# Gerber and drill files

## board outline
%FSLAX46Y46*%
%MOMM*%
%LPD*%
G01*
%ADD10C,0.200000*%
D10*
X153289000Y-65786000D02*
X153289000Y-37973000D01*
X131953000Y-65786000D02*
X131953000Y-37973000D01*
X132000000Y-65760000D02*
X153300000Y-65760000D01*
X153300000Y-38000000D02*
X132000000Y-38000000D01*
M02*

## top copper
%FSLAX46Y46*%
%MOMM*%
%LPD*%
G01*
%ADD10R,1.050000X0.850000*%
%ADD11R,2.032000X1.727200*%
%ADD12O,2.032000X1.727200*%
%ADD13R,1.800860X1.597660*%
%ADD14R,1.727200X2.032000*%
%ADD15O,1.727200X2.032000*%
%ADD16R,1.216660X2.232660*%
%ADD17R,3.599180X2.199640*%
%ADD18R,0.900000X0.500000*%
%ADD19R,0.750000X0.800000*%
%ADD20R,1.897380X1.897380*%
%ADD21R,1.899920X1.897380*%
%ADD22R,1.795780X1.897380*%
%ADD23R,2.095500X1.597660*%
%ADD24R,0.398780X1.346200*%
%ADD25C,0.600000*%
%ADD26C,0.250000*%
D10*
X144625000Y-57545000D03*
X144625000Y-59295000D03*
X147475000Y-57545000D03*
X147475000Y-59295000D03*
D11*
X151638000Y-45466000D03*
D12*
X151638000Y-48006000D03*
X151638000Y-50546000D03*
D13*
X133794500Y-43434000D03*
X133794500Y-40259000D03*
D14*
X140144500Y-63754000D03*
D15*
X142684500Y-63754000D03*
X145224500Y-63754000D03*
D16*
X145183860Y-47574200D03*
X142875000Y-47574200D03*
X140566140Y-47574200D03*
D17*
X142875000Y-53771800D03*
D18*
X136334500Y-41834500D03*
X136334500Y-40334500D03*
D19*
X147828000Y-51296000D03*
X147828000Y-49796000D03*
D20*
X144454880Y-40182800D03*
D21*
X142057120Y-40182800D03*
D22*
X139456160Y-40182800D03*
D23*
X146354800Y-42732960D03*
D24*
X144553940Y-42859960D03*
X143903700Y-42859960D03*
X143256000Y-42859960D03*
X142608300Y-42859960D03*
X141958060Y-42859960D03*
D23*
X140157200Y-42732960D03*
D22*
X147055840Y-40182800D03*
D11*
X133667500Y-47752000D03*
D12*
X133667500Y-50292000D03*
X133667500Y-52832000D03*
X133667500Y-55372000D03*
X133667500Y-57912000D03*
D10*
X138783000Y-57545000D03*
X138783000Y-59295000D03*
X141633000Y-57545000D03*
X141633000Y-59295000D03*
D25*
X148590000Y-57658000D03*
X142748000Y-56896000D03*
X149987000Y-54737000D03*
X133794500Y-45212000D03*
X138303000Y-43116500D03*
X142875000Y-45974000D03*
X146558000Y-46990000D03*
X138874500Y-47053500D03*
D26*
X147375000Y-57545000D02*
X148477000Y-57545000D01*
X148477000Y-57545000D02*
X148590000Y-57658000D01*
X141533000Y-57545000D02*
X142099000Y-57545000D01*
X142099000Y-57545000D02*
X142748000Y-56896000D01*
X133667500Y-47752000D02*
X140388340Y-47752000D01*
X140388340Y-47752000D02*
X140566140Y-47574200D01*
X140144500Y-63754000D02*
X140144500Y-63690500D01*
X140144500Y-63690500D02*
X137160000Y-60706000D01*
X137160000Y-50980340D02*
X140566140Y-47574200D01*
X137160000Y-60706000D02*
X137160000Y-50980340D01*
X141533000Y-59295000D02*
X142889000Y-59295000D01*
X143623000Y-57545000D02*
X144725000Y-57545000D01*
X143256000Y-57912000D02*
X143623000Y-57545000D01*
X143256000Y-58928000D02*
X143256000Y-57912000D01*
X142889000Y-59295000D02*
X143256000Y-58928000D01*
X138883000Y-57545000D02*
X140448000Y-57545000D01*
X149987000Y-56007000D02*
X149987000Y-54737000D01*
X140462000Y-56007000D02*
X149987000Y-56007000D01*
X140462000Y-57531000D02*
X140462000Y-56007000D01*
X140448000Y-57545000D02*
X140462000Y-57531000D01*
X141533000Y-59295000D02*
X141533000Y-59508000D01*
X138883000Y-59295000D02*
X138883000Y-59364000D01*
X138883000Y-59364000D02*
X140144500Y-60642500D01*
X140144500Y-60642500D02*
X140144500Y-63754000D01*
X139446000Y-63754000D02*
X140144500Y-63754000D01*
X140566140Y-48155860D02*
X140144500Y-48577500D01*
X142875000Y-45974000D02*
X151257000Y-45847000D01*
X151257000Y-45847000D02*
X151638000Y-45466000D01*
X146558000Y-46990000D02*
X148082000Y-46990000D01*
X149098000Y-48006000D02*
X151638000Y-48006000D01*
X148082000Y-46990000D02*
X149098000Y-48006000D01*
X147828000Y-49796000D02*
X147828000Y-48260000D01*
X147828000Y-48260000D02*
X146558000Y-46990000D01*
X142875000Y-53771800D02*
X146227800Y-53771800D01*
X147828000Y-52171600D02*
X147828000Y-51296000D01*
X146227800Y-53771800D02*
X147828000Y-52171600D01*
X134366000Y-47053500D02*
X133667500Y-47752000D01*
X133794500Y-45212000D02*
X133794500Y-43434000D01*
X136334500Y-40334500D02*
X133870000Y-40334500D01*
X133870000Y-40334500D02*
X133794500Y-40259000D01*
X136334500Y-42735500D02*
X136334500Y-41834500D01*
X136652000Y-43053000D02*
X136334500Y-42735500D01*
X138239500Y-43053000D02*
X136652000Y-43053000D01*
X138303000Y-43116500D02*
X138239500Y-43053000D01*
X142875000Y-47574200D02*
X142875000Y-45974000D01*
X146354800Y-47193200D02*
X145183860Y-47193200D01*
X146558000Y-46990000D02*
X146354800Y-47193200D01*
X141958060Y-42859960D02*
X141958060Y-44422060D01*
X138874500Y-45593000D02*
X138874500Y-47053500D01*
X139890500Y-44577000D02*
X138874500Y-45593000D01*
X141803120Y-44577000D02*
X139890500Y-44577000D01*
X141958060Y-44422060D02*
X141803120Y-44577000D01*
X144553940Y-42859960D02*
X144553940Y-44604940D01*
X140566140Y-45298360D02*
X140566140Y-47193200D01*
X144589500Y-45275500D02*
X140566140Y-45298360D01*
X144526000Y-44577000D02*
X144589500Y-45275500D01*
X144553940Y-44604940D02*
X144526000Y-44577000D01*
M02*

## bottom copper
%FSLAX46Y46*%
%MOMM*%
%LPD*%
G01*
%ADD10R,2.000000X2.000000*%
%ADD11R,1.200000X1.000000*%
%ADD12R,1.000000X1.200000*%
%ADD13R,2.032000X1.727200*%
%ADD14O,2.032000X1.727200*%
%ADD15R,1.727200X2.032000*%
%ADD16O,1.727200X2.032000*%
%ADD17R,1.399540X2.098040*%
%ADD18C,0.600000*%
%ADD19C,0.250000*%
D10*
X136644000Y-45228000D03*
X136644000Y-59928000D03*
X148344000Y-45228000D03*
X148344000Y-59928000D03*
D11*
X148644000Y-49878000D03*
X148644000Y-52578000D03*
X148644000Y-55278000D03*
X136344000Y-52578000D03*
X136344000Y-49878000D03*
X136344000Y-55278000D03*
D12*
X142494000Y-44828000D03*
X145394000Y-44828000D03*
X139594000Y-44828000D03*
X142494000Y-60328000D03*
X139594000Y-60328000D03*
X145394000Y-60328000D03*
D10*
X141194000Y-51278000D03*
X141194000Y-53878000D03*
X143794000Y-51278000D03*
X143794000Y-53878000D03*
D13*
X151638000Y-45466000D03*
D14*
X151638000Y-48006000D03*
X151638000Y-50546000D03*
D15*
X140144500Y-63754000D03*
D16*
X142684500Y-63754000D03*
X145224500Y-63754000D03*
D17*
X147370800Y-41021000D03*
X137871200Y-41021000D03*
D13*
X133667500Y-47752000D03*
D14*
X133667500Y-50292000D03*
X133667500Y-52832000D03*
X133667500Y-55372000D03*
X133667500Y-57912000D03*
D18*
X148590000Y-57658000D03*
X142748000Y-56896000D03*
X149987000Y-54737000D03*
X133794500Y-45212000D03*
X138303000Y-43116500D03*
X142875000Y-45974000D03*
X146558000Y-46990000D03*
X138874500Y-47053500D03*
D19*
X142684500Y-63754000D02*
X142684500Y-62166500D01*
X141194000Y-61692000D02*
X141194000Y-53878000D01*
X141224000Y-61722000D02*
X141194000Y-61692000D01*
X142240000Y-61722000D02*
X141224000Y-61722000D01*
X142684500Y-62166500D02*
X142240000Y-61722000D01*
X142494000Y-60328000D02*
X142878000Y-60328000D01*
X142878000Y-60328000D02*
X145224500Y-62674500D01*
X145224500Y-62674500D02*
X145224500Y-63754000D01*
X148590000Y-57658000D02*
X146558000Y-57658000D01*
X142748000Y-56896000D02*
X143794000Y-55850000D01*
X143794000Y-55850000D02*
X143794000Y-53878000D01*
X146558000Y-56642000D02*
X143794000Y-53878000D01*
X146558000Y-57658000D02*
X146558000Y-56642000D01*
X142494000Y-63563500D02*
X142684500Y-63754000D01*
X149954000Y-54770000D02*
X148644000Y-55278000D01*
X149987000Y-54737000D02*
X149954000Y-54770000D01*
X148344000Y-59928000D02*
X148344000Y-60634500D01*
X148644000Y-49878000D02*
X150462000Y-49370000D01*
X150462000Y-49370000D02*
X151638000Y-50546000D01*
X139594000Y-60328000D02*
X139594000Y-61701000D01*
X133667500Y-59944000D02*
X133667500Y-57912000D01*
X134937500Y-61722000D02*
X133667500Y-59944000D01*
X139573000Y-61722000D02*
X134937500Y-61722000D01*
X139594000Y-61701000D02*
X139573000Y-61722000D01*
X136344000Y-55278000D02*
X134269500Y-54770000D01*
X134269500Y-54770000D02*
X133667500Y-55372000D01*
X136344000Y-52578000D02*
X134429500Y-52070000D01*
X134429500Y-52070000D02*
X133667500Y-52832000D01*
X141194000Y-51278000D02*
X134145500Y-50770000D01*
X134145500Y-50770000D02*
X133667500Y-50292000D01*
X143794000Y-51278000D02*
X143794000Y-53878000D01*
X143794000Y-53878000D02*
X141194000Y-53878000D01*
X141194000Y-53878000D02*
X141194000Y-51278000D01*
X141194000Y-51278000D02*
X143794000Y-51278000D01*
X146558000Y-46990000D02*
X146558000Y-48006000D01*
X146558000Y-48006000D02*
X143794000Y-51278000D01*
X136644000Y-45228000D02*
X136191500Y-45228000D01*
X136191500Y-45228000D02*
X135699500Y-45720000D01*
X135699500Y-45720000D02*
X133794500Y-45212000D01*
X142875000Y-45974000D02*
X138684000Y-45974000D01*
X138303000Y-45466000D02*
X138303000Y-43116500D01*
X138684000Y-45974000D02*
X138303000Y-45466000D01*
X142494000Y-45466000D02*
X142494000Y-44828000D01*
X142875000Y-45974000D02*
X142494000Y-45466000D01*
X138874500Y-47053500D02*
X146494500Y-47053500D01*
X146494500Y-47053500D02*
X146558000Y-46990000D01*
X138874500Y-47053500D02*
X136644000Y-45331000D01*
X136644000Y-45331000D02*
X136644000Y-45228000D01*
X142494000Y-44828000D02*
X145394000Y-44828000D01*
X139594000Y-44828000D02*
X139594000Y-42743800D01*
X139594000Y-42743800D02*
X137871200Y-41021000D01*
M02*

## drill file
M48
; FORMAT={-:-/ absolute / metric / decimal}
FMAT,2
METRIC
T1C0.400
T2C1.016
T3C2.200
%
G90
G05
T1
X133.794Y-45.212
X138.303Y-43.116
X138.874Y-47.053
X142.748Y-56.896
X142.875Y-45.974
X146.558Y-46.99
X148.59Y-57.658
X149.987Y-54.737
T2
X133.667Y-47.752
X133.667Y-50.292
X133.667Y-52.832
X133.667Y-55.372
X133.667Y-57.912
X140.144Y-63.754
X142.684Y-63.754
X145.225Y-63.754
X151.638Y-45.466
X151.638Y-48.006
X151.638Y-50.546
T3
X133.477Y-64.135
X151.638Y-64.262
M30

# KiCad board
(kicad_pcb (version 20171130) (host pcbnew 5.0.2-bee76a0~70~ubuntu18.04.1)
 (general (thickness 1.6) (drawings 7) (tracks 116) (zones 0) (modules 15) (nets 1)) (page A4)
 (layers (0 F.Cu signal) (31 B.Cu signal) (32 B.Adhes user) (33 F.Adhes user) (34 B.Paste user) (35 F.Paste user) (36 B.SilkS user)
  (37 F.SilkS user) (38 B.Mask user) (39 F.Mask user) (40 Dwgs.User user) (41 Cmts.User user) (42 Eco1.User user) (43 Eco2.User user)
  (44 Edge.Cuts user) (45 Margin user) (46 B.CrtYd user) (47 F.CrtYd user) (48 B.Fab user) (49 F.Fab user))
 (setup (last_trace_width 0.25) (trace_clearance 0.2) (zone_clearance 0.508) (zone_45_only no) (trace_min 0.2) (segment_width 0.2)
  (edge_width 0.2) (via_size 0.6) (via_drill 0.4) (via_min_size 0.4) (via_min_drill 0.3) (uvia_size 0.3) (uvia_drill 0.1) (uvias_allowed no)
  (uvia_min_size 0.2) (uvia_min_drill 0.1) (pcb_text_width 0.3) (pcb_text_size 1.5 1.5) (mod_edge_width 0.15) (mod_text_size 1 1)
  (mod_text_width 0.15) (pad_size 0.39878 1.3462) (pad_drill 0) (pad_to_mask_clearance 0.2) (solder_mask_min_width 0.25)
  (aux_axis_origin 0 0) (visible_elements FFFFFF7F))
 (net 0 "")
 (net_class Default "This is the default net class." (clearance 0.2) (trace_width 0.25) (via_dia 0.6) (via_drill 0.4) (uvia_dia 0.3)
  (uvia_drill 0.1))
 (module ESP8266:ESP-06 (layer B.Cu) (at 142.494 52.578 270)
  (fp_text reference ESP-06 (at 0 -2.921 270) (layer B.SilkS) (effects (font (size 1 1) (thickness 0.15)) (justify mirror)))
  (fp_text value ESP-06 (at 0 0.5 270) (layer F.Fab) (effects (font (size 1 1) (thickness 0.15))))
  (pad GND smd rect (at -7.35 5.85 270) (size 2 2) (layers B.Cu B.Paste B.Mask))
  (pad GP5 smd rect (at 7.35 5.85 270) (size 2 2) (layers B.Cu B.Paste B.Mask))
  (pad GP16 smd rect (at -7.35 -5.85 270) (size 2 2) (layers B.Cu B.Paste B.Mask))
  (pad GP15 smd rect (at 7.35 -5.85 270) (size 2 2) (layers B.Cu B.Paste B.Mask))
  (pad GP14 smd rect (at -2.7 -6.15 270) (size 1 1.2) (layers B.Cu B.Paste B.Mask))
  (pad GP12 smd rect (at 0 -6.15 270) (size 1 1.2) (layers B.Cu B.Paste B.Mask))
  (pad GP13 smd rect (at 2.7 -6.15 270) (size 1 1.2) (layers B.Cu B.Paste B.Mask))
  (pad TX smd rect (at 0 6.15 270) (size 1 1.2) (layers B.Cu B.Paste B.Mask))
  (pad RST smd rect (at -2.7 6.15 270) (size 1 1.2) (layers B.Cu B.Paste B.Mask))
  (pad RX smd rect (at 2.7 6.15 270) (size 1 1.2) (layers B.Cu B.Paste B.Mask))
  (pad 3.3 smd rect (at -7.75 0 270) (size 1.2 1) (layers B.Cu B.Paste B.Mask))
  (pad CHPD smd rect (at -7.75 -2.9 270) (size 1.2 1) (layers B.Cu B.Paste B.Mask))
  (pad ANT smd rect (at -7.75 2.9 270) (size 1.2 1) (layers B.Cu B.Paste B.Mask))
  (pad GP2 smd rect (at 7.75 0 270) (size 1.2 1) (layers B.Cu B.Paste B.Mask))
  (pad GP0 smd rect (at 7.75 2.9 270) (size 1.2 1) (layers B.Cu B.Paste B.Mask))
  (pad GP4 smd rect (at 7.75 -2.9 270) (size 1.2 1) (layers B.Cu B.Paste B.Mask))
  (pad GND smd rect (at -1.3 1.3 270) (size 2 2) (layers B.Cu B.Paste B.Mask))
  (pad GND smd rect (at 1.3 1.3 270) (size 2 2) (layers B.Cu B.Paste B.Mask))
  (pad GND smd rect (at -1.3 -1.3 270) (size 2 2) (layers B.Cu B.Paste B.Mask))
  (pad GND smd rect (at 1.3 -1.3 270) (size 2 2) (layers B.Cu B.Paste B.Mask)))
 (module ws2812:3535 (layer F.Cu) (at 146.05 58.42 180)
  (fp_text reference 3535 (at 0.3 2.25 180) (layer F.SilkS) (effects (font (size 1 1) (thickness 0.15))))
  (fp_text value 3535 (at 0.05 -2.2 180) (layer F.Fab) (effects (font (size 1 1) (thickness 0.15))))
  (pad IN smd rect (at 1.325 0.875 180) (size 1.05 0.85) (drill (offset 0.1 0)) (layers F.Cu F.Paste F.Mask))
  (pad VDD smd rect (at 1.325 -0.875 180) (size 1.05 0.85) (drill (offset 0.1 0)) (layers F.Cu F.Paste F.Mask))
  (pad VSS smd rect (at -1.325 0.875 180) (size 1.05 0.85) (drill (offset -0.1 0)) (layers F.Cu F.Paste F.Mask))
  (pad OUT smd rect (at -1.325 -0.875 180) (size 1.05 0.85) (drill (offset -0.1 0)) (layers F.Cu F.Paste F.Mask)))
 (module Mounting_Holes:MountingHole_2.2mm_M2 (layer F.Cu) (at 133.477 64.135)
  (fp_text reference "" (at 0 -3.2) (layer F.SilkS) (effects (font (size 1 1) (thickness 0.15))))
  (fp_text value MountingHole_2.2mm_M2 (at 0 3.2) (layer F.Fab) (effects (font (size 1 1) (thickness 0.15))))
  (pad 1 np_thru_hole circle (at 0 0) (size 2.2 2.2) (drill 2.2) (layers *.Cu *.Mask F.SilkS)))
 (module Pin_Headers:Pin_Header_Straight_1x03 (layer F.Cu) (at 151.638 45.466)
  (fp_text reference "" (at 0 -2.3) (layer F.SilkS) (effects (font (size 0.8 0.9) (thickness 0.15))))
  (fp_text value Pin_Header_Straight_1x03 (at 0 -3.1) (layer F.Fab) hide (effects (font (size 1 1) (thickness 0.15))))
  (pad 1 thru_hole rect (at 0 0) (size 2.032 1.7272) (drill 1.016) (layers *.Cu *.Mask F.SilkS))
  (pad 2 thru_hole oval (at 0 2.54) (size 2.032 1.7272) (drill 1.016) (layers *.Cu *.Mask F.SilkS))
  (pad 3 thru_hole oval (at 0 5.08) (size 2.032 1.7272) (drill 1.016) (layers *.Cu *.Mask F.SilkS)))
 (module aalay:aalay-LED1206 (layer F.Cu) (at 133.7945 41.8465 90)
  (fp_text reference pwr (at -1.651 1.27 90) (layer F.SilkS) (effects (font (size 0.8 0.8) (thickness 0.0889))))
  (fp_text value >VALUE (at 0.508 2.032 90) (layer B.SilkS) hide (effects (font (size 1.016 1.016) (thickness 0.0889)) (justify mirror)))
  (pad A smd rect (at -1.5875 0 90) (size 1.59766 1.80086) (layers F.Cu F.Paste F.Mask))
  (pad K smd rect (at 1.5875 0 90) (size 1.59766 1.80086) (layers F.Cu F.Paste F.Mask)))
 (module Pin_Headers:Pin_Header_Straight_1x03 (layer F.Cu) (at 140.1445 63.754 90)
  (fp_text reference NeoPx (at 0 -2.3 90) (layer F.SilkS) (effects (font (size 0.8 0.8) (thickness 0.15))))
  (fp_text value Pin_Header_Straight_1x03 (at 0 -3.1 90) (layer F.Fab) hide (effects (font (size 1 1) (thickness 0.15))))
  (pad 1 thru_hole rect (at 0 0 90) (size 2.032 1.7272) (drill 1.016) (layers *.Cu *.Mask F.SilkS))
  (pad 2 thru_hole oval (at 0 2.54 90) (size 2.032 1.7272) (drill 1.016) (layers *.Cu *.Mask F.SilkS))
  (pad 3 thru_hole oval (at 0 5.08 90) (size 2.032 1.7272) (drill 1.016) (layers *.Cu *.Mask F.SilkS)))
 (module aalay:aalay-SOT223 (layer F.Cu) (at 142.875 50.673 180)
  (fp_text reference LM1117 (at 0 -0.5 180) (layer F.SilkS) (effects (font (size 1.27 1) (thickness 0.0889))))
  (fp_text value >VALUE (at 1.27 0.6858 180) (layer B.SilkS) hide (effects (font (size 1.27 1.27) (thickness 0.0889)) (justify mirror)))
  (pad GND smd rect (at -2.30886 3.0988 180) (size 1.21666 2.23266) (layers F.Cu F.Paste F.Mask))
  (pad OUT smd rect (at 0 3.0988 180) (size 1.21666 2.23266) (layers F.Cu F.Paste F.Mask))
  (pad IN smd rect (at 2.30886 3.0988 180) (size 1.21666 2.23266) (layers F.Cu F.Paste F.Mask))
  (pad OUT smd rect (at 0 -3.0988 180) (size 3.59918 2.19964) (layers F.Cu F.Paste F.Mask)))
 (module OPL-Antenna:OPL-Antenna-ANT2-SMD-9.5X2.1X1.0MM (layer B.Cu) (at 142.621 41.021 180)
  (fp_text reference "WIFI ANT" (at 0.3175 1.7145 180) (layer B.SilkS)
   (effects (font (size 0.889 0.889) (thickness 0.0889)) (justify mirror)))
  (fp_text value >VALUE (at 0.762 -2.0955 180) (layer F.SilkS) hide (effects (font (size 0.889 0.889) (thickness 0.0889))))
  (pad 1 smd rect (at -4.7498 0 180) (size 1.39954 2.09804) (layers B.Cu B.Paste B.Mask))
  (pad 2 smd rect (at 4.7498 0 180) (size 1.39954 2.09804) (layers B.Cu B.Paste B.Mask)))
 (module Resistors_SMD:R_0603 (layer F.Cu) (at 136.3345 41.0845 90)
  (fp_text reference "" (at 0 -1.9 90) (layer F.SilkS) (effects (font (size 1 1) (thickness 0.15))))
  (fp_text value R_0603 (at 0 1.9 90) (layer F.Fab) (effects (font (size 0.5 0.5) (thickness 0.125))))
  (pad 1 smd rect (at -0.75 0 90) (size 0.5 0.9) (layers F.Cu F.Paste F.Mask))
  (pad 2 smd rect (at 0.75 0 90) (size 0.5 0.9) (layers F.Cu F.Paste F.Mask)))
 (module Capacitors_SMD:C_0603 (layer F.Cu) (at 147.828 50.546 90)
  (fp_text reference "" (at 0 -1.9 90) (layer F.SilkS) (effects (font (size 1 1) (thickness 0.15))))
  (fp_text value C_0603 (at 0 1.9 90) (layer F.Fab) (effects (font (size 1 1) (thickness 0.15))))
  (pad 1 smd rect (at -0.75 0 90) (size 0.8 0.75) (layers F.Cu F.Paste F.Mask))
  (pad 2 smd rect (at 0.75 0 90) (size 0.8 0.75) (layers F.Cu F.Paste F.Mask)))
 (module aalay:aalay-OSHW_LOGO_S (layer F.Cu) (at 150.622 39.878)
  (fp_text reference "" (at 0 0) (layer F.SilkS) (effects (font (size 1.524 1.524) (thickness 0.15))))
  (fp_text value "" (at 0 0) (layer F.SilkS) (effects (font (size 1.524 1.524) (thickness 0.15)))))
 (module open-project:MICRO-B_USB (layer F.Cu) (at 143.256 38.735 180)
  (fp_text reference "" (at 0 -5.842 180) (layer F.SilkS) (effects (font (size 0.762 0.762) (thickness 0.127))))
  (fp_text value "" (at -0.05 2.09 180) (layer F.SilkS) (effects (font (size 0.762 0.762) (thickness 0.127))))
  (pad "" smd rect (at -1.19888 -1.4478 180) (size 1.89738 1.89738) (layers F.Cu F.Paste F.Mask))
  (pad "" smd rect (at 1.19888 -1.4478 180) (size 1.89992 1.89738) (layers F.Cu F.Paste F.Mask))
  (pad "" smd rect (at 3.79984 -1.4478 180) (size 1.79578 1.89738) (layers F.Cu F.Paste F.Mask))
  (pad "" smd rect (at -3.0988 -3.99796 180) (size 2.0955 1.59766) (layers F.Cu F.Paste F.Mask))
  (pad +5 smd rect (at -1.29794 -4.12496 180) (size 0.39878 1.3462) (layers F.Cu F.Paste F.Mask) (clearance 0.2032))
  (pad 2 smd rect (at -0.6477 -4.12496 180) (size 0.39878 1.3462) (layers F.Cu F.Paste F.Mask) (clearance 0.2032))
  (pad 3 smd rect (at 0 -4.12496 180) (size 0.39878 1.3462) (layers F.Cu F.Paste F.Mask) (clearance 0.2032))
  (pad 4 smd rect (at 0.6477 -4.12496 180) (size 0.39878 1.3462) (layers F.Cu F.Paste F.Mask) (clearance 0.2032))
  (pad GND smd rect (at 1.29794 -4.12496 180) (size 0.39878 1.3462) (layers F.Cu F.Paste F.Mask) (clearance 0.2032))
  (pad "" smd rect (at 3.0988 -3.99796 180) (size 2.0955 1.59766) (layers F.Cu F.Paste F.Mask))
  (pad "" smd rect (at -3.79984 -1.4478 180) (size 1.79578 1.89738) (layers F.Cu F.Paste F.Mask)))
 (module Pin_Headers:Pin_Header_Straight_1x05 (layer F.Cu) (at 133.6675 47.752)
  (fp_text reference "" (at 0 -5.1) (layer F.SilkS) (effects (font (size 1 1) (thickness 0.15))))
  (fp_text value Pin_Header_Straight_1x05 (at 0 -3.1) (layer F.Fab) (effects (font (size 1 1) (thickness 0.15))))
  (pad 1 thru_hole rect (at 0 0) (size 2.032 1.7272) (drill 1.016) (layers *.Cu *.Mask F.SilkS))
  (pad 2 thru_hole oval (at 0 2.54) (size 2.032 1.7272) (drill 1.016) (layers *.Cu *.Mask F.SilkS))
  (pad 3 thru_hole oval (at 0 5.08) (size 2.032 1.7272) (drill 1.016) (layers *.Cu *.Mask F.SilkS))
  (pad 4 thru_hole oval (at 0 7.62) (size 2.032 1.7272) (drill 1.016) (layers *.Cu *.Mask F.SilkS))
  (pad 5 thru_hole oval (at 0 10.16) (size 2.032 1.7272) (drill 1.016) (layers *.Cu *.Mask F.SilkS)))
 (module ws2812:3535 (layer F.Cu) (at 140.208 58.42 180)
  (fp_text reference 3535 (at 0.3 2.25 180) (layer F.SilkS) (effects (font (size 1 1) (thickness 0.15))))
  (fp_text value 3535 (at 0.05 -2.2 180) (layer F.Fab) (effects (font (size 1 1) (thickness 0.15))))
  (pad IN smd rect (at 1.325 0.875 180) (size 1.05 0.85) (drill (offset 0.1 0)) (layers F.Cu F.Paste F.Mask))
  (pad VDD smd rect (at 1.325 -0.875 180) (size 1.05 0.85) (drill (offset 0.1 0)) (layers F.Cu F.Paste F.Mask))
  (pad VSS smd rect (at -1.325 0.875 180) (size 1.05 0.85) (drill (offset -0.1 0)) (layers F.Cu F.Paste F.Mask))
  (pad OUT smd rect (at -1.325 -0.875 180) (size 1.05 0.85) (drill (offset -0.1 0)) (layers F.Cu F.Paste F.Mask)))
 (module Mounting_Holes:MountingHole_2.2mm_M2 (layer F.Cu) (at 151.638 64.262)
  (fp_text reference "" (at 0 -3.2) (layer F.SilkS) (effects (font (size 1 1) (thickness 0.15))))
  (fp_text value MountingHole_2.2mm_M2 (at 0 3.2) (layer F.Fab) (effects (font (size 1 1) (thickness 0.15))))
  (pad 1 np_thru_hole circle (at 0 0) (size 2.2 2.2) (drill 2.2) (layers *.Cu *.Mask F.SilkS)))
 (gr_line (start 153.289 65.786) (end 153.289 37.973) (angle 90) (layer Edge.Cuts) (width 0.2))
 (gr_line (start 131.953 65.786) (end 131.953 37.973) (angle 90) (layer Edge.Cuts) (width 0.2))
 (gr_line (start 132 65.76) (end 153.3 65.76) (angle 90) (layer Edge.Cuts) (width 0.2))
 (gr_line (start 153.3 38) (end 132 38) (angle 90) (layer Edge.Cuts) (width 0.2))
 (segment (start 142.6845 63.754) (end 142.6845 62.1665) (width 0.25) (layer B.Cu) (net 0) (status 400000))
 (segment (start 141.194 61.692) (end 141.194 53.878) (width 0.25) (layer B.Cu) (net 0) (status 800000))
 (segment (start 141.224 61.722) (end 141.194 61.692) (width 0.25) (layer B.Cu) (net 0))
 (segment (start 142.24 61.722) (end 141.224 61.722) (width 0.25) (layer B.Cu) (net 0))
 (segment (start 142.6845 62.1665) (end 142.24 61.722) (width 0.25) (layer B.Cu) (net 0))
 (segment (start 142.494 60.328) (end 142.878 60.328) (width 0.25) (layer B.Cu) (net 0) (status C00000))
 (segment (start 142.878 60.328) (end 145.2245 62.6745) (width 0.25) (layer B.Cu) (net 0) (status 400000))
 (segment (start 145.2245 62.6745) (end 145.2245 63.754) (width 0.25) (layer B.Cu) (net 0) (status 800000))
 (segment (start 147.375 57.545) (end 148.477 57.545) (width 0.25) (layer F.Cu) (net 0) (status 400000))
 (segment (start 148.59 57.658) (end 146.558 57.658) (width 0.25) (layer B.Cu) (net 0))
 (via (at 148.59 57.658) (size 0.6) (drill 0.4) (layers F.Cu B.Cu) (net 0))
 (segment (start 148.477 57.545) (end 148.59 57.658) (width 0.25) (layer F.Cu) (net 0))
 (segment (start 141.533 57.545) (end 142.099 57.545) (width 0.25) (layer F.Cu) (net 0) (status C00000))
 (segment (start 142.099 57.545) (end 142.748 56.896) (width 0.25) (layer F.Cu) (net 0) (status 400000))
 (via (at 142.748 56.896) (size 0.6) (drill 0.4) (layers F.Cu B.Cu) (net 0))
 (segment (start 142.748 56.896) (end 143.794 55.85) (width 0.25) (layer B.Cu) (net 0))
 (segment (start 143.794 55.85) (end 143.794 53.878) (width 0.25) (layer B.Cu) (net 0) (status 800000))
 (segment (start 133.6675 47.752) (end 140.38834 47.752) (width 0.25) (layer F.Cu) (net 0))
 (segment (start 140.38834 47.752) (end 140.56614 47.5742) (width 0.25) (layer F.Cu) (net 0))
 (segment (start 140.1445 63.754) (end 140.1445 63.6905) (width 0.25) (layer F.Cu) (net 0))
 (segment (start 140.1445 63.6905) (end 137.16 60.706) (width 0.25) (layer F.Cu) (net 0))
 (segment (start 137.16 50.98034) (end 140.56614 47.5742) (width 0.25) (layer F.Cu) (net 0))
 (segment (start 137.16 60.706) (end 137.16 50.98034) (width 0.25) (layer F.Cu) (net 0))
 (segment (start 141.533 59.295) (end 142.889 59.295) (width 0.25) (layer F.Cu) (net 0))
 (segment (start 143.623 57.545) (end 144.725 57.545) (width 0.25) (layer F.Cu) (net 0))
 (segment (start 143.256 57.912) (end 143.623 57.545) (width 0.25) (layer F.Cu) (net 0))
 (segment (start 143.256 58.928) (end 143.256 57.912) (width 0.25) (layer F.Cu) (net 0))
 (segment (start 142.889 59.295) (end 143.256 58.928) (width 0.25) (layer F.Cu) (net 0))
 (segment (start 146.558 56.642) (end 143.794 53.878) (width 0.25) (layer B.Cu) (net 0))
 (segment (start 146.558 57.658) (end 146.558 56.642) (width 0.25) (layer B.Cu) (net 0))
 (segment (start 142.494 63.5635) (end 142.6845 63.754) (width 0.25) (layer B.Cu) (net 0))
 (segment (start 138.883 57.545) (end 140.448 57.545) (width 0.25) (layer F.Cu) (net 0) (status 10))
 (segment (start 149.954 54.77) (end 148.644 55.278) (width 0.25) (layer B.Cu) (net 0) (status 20))
 (segment (start 149.987 54.737) (end 149.954 54.77) (width 0.25) (layer B.Cu) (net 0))
 (via (at 149.987 54.737) (size 0.6) (drill 0.4) (layers F.Cu B.Cu) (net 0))
 (segment (start 149.987 56.007) (end 149.987 54.737) (width 0.25) (layer F.Cu) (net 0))
 (segment (start 140.462 56.007) (end 149.987 56.007) (width 0.25) (layer F.Cu) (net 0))
 (segment (start 140.462 57.531) (end 140.462 56.007) (width 0.25) (layer F.Cu) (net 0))
 (segment (start 140.448 57.545) (end 140.462 57.531) (width 0.25) (layer F.Cu) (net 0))
 (segment (start 141.533 59.295) (end 141.533 59.508) (width 0.25) (layer F.Cu) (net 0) (status 30))
 (segment (start 138.883 59.295) (end 138.883 59.364) (width 0.25) (layer F.Cu) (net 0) (status 30))
 (segment (start 138.883 59.364) (end 140.1445 60.6425) (width 0.25) (layer F.Cu) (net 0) (status 10))
 (segment (start 140.1445 60.6425) (end 140.1445 63.754) (width 0.25) (layer F.Cu) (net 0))
 (segment (start 139.446 63.754) (end 140.1445 63.754) (width 0.25) (layer F.Cu) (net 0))
 (segment (start 140.56614 48.15586) (end 140.1445 48.5775) (width 0.25) (layer F.Cu) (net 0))
 (segment (start 148.344 59.928) (end 148.344 60.6345) (width 0.25) (layer B.Cu) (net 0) (status 10))
 (segment (start 148.644 49.878) (end 150.462 49.37) (width 0.25) (layer B.Cu) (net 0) (status 10))
 (segment (start 150.462 49.37) (end 151.638 50.546) (width 0.25) (layer B.Cu) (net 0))
 (segment (start 142.875 45.974) (end 151.257 45.847) (width 0.25) (layer F.Cu) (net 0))
 (segment (start 151.257 45.847) (end 151.638 45.466) (width 0.25) (layer F.Cu) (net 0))
 (segment (start 146.558 46.99) (end 148.082 46.99) (width 0.25) (layer F.Cu) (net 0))
 (segment (start 149.098 48.006) (end 151.638 48.006) (width 0.25) (layer F.Cu) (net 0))
 (segment (start 148.082 46.99) (end 149.098 48.006) (width 0.25) (layer F.Cu) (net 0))
 (segment (start 147.828 49.796) (end 147.828 48.26) (width 0.25) (layer F.Cu) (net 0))
 (segment (start 147.828 48.26) (end 146.558 46.99) (width 0.25) (layer F.Cu) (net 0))
 (segment (start 142.875 53.7718) (end 146.2278 53.7718) (width 0.25) (layer F.Cu) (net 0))
 (segment (start 147.828 52.1716) (end 147.828 51.296) (width 0.25) (layer F.Cu) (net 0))
 (segment (start 146.2278 53.7718) (end 147.828 52.1716) (width 0.25) (layer F.Cu) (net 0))
 (segment (start 139.594 60.328) (end 139.594 61.701) (width 0.25) (layer B.Cu) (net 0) (status 10))
 (segment (start 133.6675 59.944) (end 133.6675 57.912) (width 0.25) (layer B.Cu) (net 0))
 (segment (start 134.9375 61.722) (end 133.6675 59.944) (width 0.25) (layer B.Cu) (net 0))
 (segment (start 139.573 61.722) (end 134.9375 61.722) (width 0.25) (layer B.Cu) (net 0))
 (segment (start 139.594 61.701) (end 139.573 61.722) (width 0.25) (layer B.Cu) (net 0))
 (segment (start 136.344 55.278) (end 134.2695 54.77) (width 0.25) (layer B.Cu) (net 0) (status 10))
 (segment (start 134.2695 54.77) (end 133.6675 55.372) (width 0.25) (layer B.Cu) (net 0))
 (segment (start 136.344 52.578) (end 134.4295 52.07) (width 0.25) (layer B.Cu) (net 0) (status 10))
 (segment (start 134.4295 52.07) (end 133.6675 52.832) (width 0.25) (layer B.Cu) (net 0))
 (segment (start 141.194 51.278) (end 134.1455 50.77) (width 0.25) (layer B.Cu) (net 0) (status 10))
 (segment (start 134.1455 50.77) (end 133.6675 50.292) (width 0.25) (layer B.Cu) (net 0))
 (segment (start 134.366 47.0535) (end 133.6675 47.752) (width 0.25) (layer F.Cu) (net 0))
 (segment (start 143.794 51.278) (end 143.794 53.878) (width 0.25) (layer B.Cu) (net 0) (status 30))
 (segment (start 143.794 53.878) (end 141.194 53.878) (width 0.25) (layer B.Cu) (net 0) (status 30))
 (segment (start 141.194 53.878) (end 141.194 51.278) (width 0.25) (layer B.Cu) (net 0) (status 30))
 (segment (start 141.194 51.278) (end 143.794 51.278) (width 0.25) (layer B.Cu) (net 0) (status 30))
 (segment (start 146.558 46.99) (end 146.558 48.006) (width 0.25) (layer B.Cu) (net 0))
 (segment (start 146.558 48.006) (end 143.794 51.278) (width 0.25) (layer B.Cu) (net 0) (status 20))
 (segment (start 136.644 45.228) (end 136.1915 45.228) (width 0.25) (layer B.Cu) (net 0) (status 30))
 (segment (start 136.1915 45.228) (end 135.6995 45.72) (width 0.25) (layer B.Cu) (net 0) (status 30))
 (segment (start 135.6995 45.72) (end 133.7945 45.212) (width 0.25) (layer B.Cu) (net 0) (status 10))
 (via (at 133.7945 45.212) (size 0.6) (drill 0.4) (layers F.Cu B.Cu) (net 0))
 (segment (start 133.7945 45.212) (end 133.7945 43.434) (width 0.25) (layer F.Cu) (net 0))
 (segment (start 136.3345 40.3345) (end 133.87 40.3345) (width 0.25) (layer F.Cu) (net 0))
 (segment (start 133.87 40.3345) (end 133.7945 40.259) (width 0.25) (layer F.Cu) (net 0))
 (segment (start 142.875 45.974) (end 138.684 45.974) (width 0.25) (layer B.Cu) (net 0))
 (segment (start 136.3345 42.7355) (end 136.3345 41.8345) (width 0.25) (layer F.Cu) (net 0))
 (segment (start 136.652 43.053) (end 136.3345 42.7355) (width 0.25) (layer F.Cu) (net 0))
 (segment (start 138.2395 43.053) (end 136.652 43.053) (width 0.25) (layer F.Cu) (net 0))
 (segment (start 138.303 43.1165) (end 138.2395 43.053) (width 0.25) (layer F.Cu) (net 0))
 (via (at 138.303 43.1165) (size 0.6) (drill 0.4) (layers F.Cu B.Cu) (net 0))
 (segment (start 138.303 45.466) (end 138.303 43.1165) (width 0.25) (layer B.Cu) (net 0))
 (segment (start 138.684 45.974) (end 138.303 45.466) (width 0.25) (layer B.Cu) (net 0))
 (segment (start 142.875 47.5742) (end 142.875 45.974) (width 0.25) (layer F.Cu) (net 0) (status 10))
 (segment (start 142.494 45.466) (end 142.494 44.828) (width 0.25) (layer B.Cu) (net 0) (status 20))
 (segment (start 142.875 45.974) (end 142.494 45.466) (width 0.25) (layer B.Cu) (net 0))
 (via (at 142.875 45.974) (size 0.6) (drill 0.4) (layers F.Cu B.Cu) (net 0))
 (segment (start 138.8745 47.0535) (end 146.4945 47.0535) (width 0.25) (layer B.Cu) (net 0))
 (segment (start 146.3548 47.1932) (end 145.18386 47.1932) (width 0.25) (layer F.Cu) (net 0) (status 20))
 (segment (start 146.558 46.99) (end 146.3548 47.1932) (width 0.25) (layer F.Cu) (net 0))
 (via (at 146.558 46.99) (size 0.6) (drill 0.4) (layers F.Cu B.Cu) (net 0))
 (segment (start 146.4945 47.0535) (end 146.558 46.99) (width 0.25) (layer B.Cu) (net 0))
 (segment (start 141.95806 42.85996) (end 141.95806 44.42206) (width 0.25) (layer F.Cu) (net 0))
 (segment (start 138.8745 47.0535) (end 136.644 45.331) (width 0.25) (layer B.Cu) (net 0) (status 20))
 (via (at 138.8745 47.0535) (size 0.6) (drill 0.4) (layers F.Cu B.Cu) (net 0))
 (segment (start 138.8745 45.593) (end 138.8745 47.0535) (width 0.25) (layer F.Cu) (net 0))
 (segment (start 139.8905 44.577) (end 138.8745 45.593) (width 0.25) (layer F.Cu) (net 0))
 (segment (start 141.80312 44.577) (end 139.8905 44.577) (width 0.25) (layer F.Cu) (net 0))
 (segment (start 141.95806 44.42206) (end 141.80312 44.577) (width 0.25) (layer F.Cu) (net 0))
 (segment (start 136.644 45.331) (end 136.644 45.228) (width 0.25) (layer B.Cu) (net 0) (status 30))
 (segment (start 144.55394 42.85996) (end 144.55394 44.60494) (width 0.25) (layer F.Cu) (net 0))
 (segment (start 140.56614 45.29836) (end 140.56614 47.1932) (width 0.25) (layer F.Cu) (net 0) (status 20))
 (segment (start 144.5895 45.2755) (end 140.56614 45.29836) (width 0.25) (layer F.Cu) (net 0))
 (segment (start 144.526 44.577) (end 144.5895 45.2755) (width 0.25) (layer F.Cu) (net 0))
 (segment (start 144.55394 44.60494) (end 144.526 44.577) (width 0.25) (layer F.Cu) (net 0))
 (segment (start 142.494 44.828) (end 145.394 44.828) (width 0.25) (layer B.Cu) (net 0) (status 30))
 (segment (start 139.594 44.828) (end 139.594 42.7438) (width 0.25) (layer B.Cu) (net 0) (status 10))
 (segment (start 139.594 42.7438) (end 137.8712 41.021) (width 0.25) (layer B.Cu) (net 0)))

